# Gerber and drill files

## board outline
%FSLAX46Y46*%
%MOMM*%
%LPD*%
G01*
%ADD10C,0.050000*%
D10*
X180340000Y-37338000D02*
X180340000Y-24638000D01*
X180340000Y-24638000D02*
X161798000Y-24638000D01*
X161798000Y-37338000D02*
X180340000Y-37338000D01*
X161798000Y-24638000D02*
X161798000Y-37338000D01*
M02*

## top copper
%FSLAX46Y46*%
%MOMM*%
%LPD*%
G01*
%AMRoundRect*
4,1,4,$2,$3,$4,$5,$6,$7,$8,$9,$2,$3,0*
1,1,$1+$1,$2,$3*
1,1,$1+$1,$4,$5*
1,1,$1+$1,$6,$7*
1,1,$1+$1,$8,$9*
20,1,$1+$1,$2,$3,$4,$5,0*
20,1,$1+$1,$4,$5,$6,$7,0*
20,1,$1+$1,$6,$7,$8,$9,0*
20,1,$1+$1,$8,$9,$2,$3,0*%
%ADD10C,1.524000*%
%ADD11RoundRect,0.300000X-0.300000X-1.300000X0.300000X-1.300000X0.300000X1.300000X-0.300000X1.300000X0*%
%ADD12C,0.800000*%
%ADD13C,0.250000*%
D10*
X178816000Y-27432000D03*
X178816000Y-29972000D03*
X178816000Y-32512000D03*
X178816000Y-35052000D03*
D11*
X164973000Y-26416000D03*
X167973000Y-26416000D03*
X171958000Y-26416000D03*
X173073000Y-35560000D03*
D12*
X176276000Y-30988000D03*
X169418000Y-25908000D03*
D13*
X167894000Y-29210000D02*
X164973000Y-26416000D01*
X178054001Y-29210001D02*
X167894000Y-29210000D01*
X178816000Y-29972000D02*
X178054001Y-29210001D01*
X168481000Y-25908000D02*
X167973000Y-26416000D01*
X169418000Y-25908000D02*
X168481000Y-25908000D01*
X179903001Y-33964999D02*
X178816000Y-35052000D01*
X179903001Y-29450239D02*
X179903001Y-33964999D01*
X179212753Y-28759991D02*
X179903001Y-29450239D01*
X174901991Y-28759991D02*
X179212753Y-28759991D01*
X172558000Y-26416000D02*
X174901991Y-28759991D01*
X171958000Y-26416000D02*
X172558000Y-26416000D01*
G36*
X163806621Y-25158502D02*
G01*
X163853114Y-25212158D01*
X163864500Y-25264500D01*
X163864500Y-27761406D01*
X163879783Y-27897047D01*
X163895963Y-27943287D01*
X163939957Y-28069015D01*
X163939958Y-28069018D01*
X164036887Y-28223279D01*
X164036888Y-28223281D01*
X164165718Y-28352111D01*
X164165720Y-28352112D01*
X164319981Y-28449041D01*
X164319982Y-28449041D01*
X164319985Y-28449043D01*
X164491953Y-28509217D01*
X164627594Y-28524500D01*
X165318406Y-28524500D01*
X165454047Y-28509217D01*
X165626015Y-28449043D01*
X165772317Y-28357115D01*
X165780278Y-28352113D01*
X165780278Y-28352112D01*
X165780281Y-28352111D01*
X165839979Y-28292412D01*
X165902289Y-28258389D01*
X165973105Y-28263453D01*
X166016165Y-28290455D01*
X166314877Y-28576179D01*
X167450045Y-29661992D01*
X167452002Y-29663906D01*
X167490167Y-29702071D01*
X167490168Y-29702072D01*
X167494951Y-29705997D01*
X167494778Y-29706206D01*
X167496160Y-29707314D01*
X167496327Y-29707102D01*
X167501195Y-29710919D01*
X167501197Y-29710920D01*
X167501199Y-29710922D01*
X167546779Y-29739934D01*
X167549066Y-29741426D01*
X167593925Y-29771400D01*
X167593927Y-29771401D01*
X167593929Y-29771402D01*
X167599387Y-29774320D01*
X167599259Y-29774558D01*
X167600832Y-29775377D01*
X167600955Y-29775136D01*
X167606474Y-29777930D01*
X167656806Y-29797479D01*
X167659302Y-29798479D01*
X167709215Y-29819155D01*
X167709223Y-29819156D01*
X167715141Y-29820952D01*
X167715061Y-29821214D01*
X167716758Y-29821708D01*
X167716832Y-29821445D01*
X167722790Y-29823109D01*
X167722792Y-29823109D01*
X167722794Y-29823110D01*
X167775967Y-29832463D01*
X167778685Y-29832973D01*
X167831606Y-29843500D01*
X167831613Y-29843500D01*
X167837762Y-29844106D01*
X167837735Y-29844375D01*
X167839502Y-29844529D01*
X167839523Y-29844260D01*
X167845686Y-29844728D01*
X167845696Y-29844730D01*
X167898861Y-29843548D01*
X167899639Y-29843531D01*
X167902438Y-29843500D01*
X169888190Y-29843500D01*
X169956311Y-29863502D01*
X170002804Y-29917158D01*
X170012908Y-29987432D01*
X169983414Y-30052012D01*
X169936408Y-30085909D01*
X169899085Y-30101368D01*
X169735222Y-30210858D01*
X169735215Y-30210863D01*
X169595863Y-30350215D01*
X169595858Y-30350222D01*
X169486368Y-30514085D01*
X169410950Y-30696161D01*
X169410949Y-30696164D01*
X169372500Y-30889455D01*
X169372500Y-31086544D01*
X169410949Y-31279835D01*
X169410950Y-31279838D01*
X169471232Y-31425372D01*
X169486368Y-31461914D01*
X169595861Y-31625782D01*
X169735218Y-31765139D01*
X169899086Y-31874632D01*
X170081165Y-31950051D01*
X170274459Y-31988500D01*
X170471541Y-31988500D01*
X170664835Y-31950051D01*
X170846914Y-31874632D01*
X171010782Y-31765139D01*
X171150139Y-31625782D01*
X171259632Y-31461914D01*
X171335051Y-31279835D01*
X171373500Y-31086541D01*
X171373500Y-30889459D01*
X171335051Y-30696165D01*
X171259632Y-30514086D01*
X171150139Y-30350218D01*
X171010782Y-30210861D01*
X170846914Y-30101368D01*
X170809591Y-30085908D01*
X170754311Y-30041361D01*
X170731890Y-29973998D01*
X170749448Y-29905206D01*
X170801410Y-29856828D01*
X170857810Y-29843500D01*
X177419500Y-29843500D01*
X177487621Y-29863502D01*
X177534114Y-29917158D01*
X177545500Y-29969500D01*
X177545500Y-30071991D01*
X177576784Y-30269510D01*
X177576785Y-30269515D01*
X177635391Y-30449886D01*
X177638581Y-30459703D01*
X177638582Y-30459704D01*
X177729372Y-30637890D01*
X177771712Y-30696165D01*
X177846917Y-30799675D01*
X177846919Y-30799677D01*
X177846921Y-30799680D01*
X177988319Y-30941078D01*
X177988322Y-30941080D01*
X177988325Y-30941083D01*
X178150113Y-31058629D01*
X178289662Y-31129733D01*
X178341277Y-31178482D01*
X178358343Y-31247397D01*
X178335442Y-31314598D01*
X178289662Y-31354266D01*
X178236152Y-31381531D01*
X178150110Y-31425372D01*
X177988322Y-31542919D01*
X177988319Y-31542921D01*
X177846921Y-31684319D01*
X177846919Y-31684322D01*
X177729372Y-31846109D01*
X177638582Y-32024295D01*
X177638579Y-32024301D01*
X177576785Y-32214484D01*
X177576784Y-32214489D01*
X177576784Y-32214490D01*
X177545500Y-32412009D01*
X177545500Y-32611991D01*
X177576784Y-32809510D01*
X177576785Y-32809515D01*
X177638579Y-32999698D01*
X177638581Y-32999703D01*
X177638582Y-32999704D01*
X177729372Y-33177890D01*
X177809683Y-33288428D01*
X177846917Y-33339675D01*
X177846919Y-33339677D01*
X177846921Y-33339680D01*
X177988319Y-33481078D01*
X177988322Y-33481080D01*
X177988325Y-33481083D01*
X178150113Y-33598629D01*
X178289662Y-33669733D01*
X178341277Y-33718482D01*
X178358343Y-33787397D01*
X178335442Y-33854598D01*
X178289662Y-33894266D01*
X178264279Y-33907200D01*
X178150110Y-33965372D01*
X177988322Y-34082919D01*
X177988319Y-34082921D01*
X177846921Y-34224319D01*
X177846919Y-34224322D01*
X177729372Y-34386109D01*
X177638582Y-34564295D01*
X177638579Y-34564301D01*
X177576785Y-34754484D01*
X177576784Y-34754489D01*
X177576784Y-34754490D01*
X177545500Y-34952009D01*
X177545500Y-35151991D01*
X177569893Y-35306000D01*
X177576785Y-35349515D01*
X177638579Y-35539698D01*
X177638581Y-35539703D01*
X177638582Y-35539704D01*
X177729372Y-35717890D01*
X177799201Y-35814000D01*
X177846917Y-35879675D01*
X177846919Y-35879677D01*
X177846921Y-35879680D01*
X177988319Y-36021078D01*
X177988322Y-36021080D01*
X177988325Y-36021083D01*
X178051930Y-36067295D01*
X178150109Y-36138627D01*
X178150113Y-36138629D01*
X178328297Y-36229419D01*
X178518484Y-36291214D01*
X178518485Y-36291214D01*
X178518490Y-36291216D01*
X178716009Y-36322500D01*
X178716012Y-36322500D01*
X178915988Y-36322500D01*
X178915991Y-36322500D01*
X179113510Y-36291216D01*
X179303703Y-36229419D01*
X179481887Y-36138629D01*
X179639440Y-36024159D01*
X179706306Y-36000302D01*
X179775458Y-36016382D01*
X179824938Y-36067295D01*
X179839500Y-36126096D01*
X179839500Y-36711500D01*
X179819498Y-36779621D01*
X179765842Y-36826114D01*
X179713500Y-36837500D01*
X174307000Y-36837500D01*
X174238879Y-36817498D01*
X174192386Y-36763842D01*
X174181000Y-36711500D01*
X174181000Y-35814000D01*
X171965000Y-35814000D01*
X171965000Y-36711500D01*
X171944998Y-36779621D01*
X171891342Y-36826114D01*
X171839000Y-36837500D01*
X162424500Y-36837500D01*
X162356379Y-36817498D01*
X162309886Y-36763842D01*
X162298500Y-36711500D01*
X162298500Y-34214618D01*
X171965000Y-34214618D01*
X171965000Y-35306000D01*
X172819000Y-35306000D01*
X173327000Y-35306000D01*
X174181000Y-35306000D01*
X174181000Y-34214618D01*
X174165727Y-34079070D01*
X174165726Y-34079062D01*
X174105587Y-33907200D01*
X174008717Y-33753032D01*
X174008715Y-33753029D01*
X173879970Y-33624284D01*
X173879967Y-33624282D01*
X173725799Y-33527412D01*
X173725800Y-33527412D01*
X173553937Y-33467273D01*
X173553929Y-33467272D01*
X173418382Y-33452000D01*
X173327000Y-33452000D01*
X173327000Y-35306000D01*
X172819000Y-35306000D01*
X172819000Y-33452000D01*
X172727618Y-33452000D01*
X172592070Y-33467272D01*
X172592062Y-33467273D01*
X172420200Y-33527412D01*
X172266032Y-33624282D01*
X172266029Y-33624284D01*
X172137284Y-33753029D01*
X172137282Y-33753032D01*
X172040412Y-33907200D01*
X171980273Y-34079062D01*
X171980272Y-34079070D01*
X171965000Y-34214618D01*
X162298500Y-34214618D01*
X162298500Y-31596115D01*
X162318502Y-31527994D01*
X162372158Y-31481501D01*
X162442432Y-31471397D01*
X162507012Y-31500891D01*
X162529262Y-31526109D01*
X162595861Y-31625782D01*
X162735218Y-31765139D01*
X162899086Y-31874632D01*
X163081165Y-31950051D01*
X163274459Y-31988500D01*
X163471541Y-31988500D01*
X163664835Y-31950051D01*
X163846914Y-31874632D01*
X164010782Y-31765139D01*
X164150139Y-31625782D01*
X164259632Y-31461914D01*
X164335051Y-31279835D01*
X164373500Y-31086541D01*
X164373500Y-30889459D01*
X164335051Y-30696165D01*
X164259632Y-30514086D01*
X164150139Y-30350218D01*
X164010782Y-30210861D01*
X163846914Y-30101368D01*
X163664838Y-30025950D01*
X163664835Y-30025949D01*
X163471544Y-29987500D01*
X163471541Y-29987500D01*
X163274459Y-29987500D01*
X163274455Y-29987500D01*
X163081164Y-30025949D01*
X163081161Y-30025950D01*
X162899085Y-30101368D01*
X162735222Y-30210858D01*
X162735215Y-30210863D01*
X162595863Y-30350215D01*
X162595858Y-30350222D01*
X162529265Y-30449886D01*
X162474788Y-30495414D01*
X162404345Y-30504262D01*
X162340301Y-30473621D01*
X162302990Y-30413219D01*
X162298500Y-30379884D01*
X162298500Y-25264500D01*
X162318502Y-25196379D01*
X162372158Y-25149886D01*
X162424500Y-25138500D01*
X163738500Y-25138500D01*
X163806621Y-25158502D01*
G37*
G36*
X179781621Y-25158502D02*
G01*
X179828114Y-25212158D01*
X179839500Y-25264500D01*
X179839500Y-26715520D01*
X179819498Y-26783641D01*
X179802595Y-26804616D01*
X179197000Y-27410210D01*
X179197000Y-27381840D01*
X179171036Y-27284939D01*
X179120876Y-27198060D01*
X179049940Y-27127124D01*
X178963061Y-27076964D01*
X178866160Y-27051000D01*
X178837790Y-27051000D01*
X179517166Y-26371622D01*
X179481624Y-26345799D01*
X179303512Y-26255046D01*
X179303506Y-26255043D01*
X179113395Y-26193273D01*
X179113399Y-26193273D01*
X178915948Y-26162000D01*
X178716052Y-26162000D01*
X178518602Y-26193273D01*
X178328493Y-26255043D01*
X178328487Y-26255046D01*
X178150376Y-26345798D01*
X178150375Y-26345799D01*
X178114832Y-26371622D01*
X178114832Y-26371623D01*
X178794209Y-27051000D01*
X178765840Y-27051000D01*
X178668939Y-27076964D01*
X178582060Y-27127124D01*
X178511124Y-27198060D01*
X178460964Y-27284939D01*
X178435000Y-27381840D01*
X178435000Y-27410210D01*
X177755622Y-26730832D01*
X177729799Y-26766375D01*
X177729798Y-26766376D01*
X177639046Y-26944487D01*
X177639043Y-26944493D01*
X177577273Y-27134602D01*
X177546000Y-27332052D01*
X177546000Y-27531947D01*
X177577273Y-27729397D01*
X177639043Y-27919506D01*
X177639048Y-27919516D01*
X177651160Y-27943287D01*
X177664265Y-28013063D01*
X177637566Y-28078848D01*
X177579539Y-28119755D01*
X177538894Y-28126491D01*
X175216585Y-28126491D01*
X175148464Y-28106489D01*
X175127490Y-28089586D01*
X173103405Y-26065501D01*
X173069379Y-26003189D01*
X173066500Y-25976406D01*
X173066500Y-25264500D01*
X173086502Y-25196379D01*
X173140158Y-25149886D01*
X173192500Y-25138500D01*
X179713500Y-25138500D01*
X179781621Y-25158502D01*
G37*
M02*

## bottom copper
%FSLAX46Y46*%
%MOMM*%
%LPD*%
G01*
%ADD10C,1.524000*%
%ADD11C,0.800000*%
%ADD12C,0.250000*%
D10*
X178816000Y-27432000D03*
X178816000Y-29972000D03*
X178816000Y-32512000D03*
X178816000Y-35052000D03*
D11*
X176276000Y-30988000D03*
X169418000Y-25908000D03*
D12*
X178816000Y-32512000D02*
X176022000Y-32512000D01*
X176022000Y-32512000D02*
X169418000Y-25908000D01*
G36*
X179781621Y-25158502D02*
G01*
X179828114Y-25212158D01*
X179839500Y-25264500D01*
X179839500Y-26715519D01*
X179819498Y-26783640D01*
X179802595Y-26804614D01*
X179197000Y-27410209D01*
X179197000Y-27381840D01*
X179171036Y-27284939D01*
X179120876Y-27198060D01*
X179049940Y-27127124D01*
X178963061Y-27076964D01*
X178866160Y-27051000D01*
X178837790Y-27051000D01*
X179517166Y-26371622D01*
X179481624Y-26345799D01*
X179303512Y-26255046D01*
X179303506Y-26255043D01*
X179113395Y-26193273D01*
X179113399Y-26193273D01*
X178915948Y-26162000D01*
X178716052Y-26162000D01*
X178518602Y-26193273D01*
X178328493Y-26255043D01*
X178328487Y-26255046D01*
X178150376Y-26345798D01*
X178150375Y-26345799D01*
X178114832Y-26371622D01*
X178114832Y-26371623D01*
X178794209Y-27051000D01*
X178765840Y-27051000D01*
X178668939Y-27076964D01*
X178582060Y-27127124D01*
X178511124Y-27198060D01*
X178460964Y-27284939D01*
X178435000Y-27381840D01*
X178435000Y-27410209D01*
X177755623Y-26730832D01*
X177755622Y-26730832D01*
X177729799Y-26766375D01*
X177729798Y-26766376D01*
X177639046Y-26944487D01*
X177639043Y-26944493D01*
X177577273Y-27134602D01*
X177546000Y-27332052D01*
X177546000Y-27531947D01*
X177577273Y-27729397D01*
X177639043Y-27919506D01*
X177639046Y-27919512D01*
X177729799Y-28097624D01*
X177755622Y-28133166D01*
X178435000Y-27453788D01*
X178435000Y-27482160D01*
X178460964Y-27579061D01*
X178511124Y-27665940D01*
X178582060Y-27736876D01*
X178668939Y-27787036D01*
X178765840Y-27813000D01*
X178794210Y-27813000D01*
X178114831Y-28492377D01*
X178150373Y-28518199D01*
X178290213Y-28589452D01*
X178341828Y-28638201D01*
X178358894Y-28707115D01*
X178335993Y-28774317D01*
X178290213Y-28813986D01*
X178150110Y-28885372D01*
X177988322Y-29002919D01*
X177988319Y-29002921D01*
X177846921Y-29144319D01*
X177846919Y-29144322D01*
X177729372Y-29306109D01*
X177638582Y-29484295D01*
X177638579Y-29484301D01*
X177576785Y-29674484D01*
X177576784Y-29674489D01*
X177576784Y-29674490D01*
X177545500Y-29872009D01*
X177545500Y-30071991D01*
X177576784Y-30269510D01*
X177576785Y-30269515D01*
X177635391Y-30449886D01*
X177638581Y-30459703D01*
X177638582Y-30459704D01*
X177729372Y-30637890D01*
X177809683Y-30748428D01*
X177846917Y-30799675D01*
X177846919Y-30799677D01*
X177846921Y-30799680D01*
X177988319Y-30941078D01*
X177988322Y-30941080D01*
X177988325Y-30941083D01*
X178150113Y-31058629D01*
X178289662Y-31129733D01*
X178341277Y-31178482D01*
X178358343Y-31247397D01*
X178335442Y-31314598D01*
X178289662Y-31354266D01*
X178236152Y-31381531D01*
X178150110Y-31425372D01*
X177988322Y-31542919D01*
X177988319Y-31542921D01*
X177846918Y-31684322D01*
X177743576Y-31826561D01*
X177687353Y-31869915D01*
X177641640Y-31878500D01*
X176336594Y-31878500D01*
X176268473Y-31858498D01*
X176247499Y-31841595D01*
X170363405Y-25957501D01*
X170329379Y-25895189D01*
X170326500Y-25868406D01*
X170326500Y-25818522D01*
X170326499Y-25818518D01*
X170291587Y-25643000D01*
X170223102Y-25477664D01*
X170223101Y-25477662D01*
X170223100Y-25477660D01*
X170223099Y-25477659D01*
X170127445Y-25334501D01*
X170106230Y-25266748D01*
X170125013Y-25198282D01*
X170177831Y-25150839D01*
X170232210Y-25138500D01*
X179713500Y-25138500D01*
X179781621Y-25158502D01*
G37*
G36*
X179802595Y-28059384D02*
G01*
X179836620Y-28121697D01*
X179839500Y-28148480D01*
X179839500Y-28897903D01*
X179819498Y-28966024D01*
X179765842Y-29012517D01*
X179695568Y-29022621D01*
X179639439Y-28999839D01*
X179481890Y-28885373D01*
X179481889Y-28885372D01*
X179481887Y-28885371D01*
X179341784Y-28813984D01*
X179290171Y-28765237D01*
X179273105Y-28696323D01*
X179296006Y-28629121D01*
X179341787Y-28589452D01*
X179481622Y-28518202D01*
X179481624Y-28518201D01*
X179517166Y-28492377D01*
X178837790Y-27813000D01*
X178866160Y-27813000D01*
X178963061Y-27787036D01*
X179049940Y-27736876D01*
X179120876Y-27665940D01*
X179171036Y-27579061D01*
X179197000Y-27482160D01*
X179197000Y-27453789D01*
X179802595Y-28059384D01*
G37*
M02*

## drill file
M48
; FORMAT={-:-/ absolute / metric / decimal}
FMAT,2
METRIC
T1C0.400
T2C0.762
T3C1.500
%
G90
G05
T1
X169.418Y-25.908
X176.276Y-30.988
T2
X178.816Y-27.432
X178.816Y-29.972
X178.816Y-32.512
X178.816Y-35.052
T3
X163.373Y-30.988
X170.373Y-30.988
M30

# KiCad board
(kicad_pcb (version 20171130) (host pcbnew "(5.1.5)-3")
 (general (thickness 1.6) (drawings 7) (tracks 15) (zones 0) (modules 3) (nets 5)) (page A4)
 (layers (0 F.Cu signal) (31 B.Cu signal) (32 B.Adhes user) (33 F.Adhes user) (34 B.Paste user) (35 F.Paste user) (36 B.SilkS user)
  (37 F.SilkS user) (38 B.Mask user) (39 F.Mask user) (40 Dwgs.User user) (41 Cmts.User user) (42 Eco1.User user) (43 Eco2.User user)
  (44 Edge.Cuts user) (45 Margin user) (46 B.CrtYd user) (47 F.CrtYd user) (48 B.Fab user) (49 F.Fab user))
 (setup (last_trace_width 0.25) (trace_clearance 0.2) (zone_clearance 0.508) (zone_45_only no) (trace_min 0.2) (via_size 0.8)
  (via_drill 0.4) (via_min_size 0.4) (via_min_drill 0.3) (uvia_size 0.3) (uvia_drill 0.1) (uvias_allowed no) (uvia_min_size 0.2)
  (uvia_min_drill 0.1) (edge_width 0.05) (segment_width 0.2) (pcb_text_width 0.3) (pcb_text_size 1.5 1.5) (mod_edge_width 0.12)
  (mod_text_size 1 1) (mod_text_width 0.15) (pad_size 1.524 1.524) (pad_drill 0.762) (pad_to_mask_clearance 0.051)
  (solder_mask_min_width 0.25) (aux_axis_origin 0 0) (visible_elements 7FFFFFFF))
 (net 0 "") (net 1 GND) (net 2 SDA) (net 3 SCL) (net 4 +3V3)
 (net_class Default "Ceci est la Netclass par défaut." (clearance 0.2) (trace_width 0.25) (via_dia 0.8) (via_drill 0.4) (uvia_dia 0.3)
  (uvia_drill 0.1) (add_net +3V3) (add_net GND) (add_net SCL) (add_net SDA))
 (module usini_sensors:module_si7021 (layer F.Cu) (at 178.816 27.432 180)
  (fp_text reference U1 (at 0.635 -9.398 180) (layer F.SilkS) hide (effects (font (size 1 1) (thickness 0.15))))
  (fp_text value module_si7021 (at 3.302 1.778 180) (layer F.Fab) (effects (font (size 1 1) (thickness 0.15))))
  (pad 4 thru_hole circle (at 0 0 180) (size 1.524 1.524) (drill 0.762) (layers *.Cu *.Mask) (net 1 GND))
  (pad 3 thru_hole circle (at 0 -2.54 180) (size 1.524 1.524) (drill 0.762) (layers *.Cu *.Mask) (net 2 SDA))
  (pad 2 thru_hole circle (at 0 -5.08 180) (size 1.524 1.524) (drill 0.762) (layers *.Cu *.Mask) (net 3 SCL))
  (pad 1 thru_hole circle (at 0 -7.62 180) (size 1.524 1.524) (drill 0.762) (layers *.Cu *.Mask) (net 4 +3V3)))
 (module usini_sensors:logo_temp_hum (layer B.Cu) (at 168.91 27.432 180)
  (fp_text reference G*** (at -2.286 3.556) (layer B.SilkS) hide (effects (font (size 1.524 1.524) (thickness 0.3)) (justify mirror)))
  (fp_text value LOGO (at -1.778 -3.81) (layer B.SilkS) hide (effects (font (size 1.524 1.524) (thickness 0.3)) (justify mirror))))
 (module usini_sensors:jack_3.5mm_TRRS (layer F.Cu) (at 168.148 30.988)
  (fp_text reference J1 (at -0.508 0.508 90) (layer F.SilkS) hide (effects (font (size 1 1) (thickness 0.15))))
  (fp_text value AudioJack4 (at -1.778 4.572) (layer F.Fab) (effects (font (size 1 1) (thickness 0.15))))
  (pad "" np_thru_hole circle (at 2.225 0) (size 1.5 1.5) (drill 1.5) (layers *.Cu *.Mask))
  (pad "" np_thru_hole circle (at -4.775 0) (size 1.5 1.5) (drill 1.5) (layers *.Cu *.Mask))
  (pad R2 smd roundrect (at -3.175 -4.572) (size 1.2 3.2) (layers F.Cu F.Paste F.Mask) (roundrect_rratio 0.25) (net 2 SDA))
  (pad R1 smd roundrect (at -0.175 -4.572) (size 1.2 3.2) (layers F.Cu F.Paste F.Mask) (roundrect_rratio 0.25) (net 3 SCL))
  (pad T smd roundrect (at 3.81 -4.572) (size 1.2 3.2) (layers F.Cu F.Paste F.Mask) (roundrect_rratio 0.25) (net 4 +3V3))
  (pad S smd roundrect (at 4.925 4.572) (size 1.2 3.2) (layers F.Cu F.Paste F.Mask) (roundrect_rratio 0.25) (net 1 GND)))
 (gr_line (start 180.34 37.338) (end 180.34 24.638) (layer Edge.Cuts) (width 0.05))
 (gr_line (start 180.34 24.638) (end 161.798 24.638) (layer Edge.Cuts) (width 0.05))
 (gr_line (start 161.798 37.338) (end 180.34 37.338) (layer Edge.Cuts) (width 0.05))
 (gr_line (start 161.798 24.638) (end 161.798 37.338) (layer Edge.Cuts) (width 0.05))
 (via (at 176.276 30.988) (size 0.8) (drill 0.4) (layers F.Cu B.Cu) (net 1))
 (segment (start 167.894 29.21) (end 164.973 26.416) (width 0.25) (layer F.Cu) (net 2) (status 20))
 (segment (start 178.054001 29.210001) (end 167.894 29.21) (width 0.25) (layer F.Cu) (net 2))
 (segment (start 178.816 29.972) (end 178.054001 29.210001) (width 0.25) (layer F.Cu) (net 2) (status 10))
 (segment (start 178.816 32.512) (end 176.022 32.512) (width 0.25) (layer B.Cu) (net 3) (status 10))
 (via (at 169.418 25.908) (size 0.8) (drill 0.4) (layers F.Cu B.Cu) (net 3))
 (segment (start 176.022 32.512) (end 169.418 25.908) (width 0.25) (layer B.Cu) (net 3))
 (segment (start 168.481 25.908) (end 167.973 26.416) (width 0.25) (layer F.Cu) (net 3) (status 30))
 (segment (start 169.418 25.908) (end 168.481 25.908) (width 0.25) (layer F.Cu) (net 3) (status 20))
 (segment (start 179.903001 33.964999) (end 178.816 35.052) (width 0.25) (layer F.Cu) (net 4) (status 20))
 (segment (start 179.903001 29.450239) (end 179.903001 33.964999) (width 0.25) (layer F.Cu) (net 4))
 (segment (start 179.212753 28.759991) (end 179.903001 29.450239) (width 0.25) (layer F.Cu) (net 4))
 (segment (start 174.901991 28.759991) (end 179.212753 28.759991) (width 0.25) (layer F.Cu) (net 4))
 (segment (start 172.558 26.416) (end 174.901991 28.759991) (width 0.25) (layer F.Cu) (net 4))
 (segment (start 171.958 26.416) (end 172.558 26.416) (width 0.25) (layer F.Cu) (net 4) (status 10))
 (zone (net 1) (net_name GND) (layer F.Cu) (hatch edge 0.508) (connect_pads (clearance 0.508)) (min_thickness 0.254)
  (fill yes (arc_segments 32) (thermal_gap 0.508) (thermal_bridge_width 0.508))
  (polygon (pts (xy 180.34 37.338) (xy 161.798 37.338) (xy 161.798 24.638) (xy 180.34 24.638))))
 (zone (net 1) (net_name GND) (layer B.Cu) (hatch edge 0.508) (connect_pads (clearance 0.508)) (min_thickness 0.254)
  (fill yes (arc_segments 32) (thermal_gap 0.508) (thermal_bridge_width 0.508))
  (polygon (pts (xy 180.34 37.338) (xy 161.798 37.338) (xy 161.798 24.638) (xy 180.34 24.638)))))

